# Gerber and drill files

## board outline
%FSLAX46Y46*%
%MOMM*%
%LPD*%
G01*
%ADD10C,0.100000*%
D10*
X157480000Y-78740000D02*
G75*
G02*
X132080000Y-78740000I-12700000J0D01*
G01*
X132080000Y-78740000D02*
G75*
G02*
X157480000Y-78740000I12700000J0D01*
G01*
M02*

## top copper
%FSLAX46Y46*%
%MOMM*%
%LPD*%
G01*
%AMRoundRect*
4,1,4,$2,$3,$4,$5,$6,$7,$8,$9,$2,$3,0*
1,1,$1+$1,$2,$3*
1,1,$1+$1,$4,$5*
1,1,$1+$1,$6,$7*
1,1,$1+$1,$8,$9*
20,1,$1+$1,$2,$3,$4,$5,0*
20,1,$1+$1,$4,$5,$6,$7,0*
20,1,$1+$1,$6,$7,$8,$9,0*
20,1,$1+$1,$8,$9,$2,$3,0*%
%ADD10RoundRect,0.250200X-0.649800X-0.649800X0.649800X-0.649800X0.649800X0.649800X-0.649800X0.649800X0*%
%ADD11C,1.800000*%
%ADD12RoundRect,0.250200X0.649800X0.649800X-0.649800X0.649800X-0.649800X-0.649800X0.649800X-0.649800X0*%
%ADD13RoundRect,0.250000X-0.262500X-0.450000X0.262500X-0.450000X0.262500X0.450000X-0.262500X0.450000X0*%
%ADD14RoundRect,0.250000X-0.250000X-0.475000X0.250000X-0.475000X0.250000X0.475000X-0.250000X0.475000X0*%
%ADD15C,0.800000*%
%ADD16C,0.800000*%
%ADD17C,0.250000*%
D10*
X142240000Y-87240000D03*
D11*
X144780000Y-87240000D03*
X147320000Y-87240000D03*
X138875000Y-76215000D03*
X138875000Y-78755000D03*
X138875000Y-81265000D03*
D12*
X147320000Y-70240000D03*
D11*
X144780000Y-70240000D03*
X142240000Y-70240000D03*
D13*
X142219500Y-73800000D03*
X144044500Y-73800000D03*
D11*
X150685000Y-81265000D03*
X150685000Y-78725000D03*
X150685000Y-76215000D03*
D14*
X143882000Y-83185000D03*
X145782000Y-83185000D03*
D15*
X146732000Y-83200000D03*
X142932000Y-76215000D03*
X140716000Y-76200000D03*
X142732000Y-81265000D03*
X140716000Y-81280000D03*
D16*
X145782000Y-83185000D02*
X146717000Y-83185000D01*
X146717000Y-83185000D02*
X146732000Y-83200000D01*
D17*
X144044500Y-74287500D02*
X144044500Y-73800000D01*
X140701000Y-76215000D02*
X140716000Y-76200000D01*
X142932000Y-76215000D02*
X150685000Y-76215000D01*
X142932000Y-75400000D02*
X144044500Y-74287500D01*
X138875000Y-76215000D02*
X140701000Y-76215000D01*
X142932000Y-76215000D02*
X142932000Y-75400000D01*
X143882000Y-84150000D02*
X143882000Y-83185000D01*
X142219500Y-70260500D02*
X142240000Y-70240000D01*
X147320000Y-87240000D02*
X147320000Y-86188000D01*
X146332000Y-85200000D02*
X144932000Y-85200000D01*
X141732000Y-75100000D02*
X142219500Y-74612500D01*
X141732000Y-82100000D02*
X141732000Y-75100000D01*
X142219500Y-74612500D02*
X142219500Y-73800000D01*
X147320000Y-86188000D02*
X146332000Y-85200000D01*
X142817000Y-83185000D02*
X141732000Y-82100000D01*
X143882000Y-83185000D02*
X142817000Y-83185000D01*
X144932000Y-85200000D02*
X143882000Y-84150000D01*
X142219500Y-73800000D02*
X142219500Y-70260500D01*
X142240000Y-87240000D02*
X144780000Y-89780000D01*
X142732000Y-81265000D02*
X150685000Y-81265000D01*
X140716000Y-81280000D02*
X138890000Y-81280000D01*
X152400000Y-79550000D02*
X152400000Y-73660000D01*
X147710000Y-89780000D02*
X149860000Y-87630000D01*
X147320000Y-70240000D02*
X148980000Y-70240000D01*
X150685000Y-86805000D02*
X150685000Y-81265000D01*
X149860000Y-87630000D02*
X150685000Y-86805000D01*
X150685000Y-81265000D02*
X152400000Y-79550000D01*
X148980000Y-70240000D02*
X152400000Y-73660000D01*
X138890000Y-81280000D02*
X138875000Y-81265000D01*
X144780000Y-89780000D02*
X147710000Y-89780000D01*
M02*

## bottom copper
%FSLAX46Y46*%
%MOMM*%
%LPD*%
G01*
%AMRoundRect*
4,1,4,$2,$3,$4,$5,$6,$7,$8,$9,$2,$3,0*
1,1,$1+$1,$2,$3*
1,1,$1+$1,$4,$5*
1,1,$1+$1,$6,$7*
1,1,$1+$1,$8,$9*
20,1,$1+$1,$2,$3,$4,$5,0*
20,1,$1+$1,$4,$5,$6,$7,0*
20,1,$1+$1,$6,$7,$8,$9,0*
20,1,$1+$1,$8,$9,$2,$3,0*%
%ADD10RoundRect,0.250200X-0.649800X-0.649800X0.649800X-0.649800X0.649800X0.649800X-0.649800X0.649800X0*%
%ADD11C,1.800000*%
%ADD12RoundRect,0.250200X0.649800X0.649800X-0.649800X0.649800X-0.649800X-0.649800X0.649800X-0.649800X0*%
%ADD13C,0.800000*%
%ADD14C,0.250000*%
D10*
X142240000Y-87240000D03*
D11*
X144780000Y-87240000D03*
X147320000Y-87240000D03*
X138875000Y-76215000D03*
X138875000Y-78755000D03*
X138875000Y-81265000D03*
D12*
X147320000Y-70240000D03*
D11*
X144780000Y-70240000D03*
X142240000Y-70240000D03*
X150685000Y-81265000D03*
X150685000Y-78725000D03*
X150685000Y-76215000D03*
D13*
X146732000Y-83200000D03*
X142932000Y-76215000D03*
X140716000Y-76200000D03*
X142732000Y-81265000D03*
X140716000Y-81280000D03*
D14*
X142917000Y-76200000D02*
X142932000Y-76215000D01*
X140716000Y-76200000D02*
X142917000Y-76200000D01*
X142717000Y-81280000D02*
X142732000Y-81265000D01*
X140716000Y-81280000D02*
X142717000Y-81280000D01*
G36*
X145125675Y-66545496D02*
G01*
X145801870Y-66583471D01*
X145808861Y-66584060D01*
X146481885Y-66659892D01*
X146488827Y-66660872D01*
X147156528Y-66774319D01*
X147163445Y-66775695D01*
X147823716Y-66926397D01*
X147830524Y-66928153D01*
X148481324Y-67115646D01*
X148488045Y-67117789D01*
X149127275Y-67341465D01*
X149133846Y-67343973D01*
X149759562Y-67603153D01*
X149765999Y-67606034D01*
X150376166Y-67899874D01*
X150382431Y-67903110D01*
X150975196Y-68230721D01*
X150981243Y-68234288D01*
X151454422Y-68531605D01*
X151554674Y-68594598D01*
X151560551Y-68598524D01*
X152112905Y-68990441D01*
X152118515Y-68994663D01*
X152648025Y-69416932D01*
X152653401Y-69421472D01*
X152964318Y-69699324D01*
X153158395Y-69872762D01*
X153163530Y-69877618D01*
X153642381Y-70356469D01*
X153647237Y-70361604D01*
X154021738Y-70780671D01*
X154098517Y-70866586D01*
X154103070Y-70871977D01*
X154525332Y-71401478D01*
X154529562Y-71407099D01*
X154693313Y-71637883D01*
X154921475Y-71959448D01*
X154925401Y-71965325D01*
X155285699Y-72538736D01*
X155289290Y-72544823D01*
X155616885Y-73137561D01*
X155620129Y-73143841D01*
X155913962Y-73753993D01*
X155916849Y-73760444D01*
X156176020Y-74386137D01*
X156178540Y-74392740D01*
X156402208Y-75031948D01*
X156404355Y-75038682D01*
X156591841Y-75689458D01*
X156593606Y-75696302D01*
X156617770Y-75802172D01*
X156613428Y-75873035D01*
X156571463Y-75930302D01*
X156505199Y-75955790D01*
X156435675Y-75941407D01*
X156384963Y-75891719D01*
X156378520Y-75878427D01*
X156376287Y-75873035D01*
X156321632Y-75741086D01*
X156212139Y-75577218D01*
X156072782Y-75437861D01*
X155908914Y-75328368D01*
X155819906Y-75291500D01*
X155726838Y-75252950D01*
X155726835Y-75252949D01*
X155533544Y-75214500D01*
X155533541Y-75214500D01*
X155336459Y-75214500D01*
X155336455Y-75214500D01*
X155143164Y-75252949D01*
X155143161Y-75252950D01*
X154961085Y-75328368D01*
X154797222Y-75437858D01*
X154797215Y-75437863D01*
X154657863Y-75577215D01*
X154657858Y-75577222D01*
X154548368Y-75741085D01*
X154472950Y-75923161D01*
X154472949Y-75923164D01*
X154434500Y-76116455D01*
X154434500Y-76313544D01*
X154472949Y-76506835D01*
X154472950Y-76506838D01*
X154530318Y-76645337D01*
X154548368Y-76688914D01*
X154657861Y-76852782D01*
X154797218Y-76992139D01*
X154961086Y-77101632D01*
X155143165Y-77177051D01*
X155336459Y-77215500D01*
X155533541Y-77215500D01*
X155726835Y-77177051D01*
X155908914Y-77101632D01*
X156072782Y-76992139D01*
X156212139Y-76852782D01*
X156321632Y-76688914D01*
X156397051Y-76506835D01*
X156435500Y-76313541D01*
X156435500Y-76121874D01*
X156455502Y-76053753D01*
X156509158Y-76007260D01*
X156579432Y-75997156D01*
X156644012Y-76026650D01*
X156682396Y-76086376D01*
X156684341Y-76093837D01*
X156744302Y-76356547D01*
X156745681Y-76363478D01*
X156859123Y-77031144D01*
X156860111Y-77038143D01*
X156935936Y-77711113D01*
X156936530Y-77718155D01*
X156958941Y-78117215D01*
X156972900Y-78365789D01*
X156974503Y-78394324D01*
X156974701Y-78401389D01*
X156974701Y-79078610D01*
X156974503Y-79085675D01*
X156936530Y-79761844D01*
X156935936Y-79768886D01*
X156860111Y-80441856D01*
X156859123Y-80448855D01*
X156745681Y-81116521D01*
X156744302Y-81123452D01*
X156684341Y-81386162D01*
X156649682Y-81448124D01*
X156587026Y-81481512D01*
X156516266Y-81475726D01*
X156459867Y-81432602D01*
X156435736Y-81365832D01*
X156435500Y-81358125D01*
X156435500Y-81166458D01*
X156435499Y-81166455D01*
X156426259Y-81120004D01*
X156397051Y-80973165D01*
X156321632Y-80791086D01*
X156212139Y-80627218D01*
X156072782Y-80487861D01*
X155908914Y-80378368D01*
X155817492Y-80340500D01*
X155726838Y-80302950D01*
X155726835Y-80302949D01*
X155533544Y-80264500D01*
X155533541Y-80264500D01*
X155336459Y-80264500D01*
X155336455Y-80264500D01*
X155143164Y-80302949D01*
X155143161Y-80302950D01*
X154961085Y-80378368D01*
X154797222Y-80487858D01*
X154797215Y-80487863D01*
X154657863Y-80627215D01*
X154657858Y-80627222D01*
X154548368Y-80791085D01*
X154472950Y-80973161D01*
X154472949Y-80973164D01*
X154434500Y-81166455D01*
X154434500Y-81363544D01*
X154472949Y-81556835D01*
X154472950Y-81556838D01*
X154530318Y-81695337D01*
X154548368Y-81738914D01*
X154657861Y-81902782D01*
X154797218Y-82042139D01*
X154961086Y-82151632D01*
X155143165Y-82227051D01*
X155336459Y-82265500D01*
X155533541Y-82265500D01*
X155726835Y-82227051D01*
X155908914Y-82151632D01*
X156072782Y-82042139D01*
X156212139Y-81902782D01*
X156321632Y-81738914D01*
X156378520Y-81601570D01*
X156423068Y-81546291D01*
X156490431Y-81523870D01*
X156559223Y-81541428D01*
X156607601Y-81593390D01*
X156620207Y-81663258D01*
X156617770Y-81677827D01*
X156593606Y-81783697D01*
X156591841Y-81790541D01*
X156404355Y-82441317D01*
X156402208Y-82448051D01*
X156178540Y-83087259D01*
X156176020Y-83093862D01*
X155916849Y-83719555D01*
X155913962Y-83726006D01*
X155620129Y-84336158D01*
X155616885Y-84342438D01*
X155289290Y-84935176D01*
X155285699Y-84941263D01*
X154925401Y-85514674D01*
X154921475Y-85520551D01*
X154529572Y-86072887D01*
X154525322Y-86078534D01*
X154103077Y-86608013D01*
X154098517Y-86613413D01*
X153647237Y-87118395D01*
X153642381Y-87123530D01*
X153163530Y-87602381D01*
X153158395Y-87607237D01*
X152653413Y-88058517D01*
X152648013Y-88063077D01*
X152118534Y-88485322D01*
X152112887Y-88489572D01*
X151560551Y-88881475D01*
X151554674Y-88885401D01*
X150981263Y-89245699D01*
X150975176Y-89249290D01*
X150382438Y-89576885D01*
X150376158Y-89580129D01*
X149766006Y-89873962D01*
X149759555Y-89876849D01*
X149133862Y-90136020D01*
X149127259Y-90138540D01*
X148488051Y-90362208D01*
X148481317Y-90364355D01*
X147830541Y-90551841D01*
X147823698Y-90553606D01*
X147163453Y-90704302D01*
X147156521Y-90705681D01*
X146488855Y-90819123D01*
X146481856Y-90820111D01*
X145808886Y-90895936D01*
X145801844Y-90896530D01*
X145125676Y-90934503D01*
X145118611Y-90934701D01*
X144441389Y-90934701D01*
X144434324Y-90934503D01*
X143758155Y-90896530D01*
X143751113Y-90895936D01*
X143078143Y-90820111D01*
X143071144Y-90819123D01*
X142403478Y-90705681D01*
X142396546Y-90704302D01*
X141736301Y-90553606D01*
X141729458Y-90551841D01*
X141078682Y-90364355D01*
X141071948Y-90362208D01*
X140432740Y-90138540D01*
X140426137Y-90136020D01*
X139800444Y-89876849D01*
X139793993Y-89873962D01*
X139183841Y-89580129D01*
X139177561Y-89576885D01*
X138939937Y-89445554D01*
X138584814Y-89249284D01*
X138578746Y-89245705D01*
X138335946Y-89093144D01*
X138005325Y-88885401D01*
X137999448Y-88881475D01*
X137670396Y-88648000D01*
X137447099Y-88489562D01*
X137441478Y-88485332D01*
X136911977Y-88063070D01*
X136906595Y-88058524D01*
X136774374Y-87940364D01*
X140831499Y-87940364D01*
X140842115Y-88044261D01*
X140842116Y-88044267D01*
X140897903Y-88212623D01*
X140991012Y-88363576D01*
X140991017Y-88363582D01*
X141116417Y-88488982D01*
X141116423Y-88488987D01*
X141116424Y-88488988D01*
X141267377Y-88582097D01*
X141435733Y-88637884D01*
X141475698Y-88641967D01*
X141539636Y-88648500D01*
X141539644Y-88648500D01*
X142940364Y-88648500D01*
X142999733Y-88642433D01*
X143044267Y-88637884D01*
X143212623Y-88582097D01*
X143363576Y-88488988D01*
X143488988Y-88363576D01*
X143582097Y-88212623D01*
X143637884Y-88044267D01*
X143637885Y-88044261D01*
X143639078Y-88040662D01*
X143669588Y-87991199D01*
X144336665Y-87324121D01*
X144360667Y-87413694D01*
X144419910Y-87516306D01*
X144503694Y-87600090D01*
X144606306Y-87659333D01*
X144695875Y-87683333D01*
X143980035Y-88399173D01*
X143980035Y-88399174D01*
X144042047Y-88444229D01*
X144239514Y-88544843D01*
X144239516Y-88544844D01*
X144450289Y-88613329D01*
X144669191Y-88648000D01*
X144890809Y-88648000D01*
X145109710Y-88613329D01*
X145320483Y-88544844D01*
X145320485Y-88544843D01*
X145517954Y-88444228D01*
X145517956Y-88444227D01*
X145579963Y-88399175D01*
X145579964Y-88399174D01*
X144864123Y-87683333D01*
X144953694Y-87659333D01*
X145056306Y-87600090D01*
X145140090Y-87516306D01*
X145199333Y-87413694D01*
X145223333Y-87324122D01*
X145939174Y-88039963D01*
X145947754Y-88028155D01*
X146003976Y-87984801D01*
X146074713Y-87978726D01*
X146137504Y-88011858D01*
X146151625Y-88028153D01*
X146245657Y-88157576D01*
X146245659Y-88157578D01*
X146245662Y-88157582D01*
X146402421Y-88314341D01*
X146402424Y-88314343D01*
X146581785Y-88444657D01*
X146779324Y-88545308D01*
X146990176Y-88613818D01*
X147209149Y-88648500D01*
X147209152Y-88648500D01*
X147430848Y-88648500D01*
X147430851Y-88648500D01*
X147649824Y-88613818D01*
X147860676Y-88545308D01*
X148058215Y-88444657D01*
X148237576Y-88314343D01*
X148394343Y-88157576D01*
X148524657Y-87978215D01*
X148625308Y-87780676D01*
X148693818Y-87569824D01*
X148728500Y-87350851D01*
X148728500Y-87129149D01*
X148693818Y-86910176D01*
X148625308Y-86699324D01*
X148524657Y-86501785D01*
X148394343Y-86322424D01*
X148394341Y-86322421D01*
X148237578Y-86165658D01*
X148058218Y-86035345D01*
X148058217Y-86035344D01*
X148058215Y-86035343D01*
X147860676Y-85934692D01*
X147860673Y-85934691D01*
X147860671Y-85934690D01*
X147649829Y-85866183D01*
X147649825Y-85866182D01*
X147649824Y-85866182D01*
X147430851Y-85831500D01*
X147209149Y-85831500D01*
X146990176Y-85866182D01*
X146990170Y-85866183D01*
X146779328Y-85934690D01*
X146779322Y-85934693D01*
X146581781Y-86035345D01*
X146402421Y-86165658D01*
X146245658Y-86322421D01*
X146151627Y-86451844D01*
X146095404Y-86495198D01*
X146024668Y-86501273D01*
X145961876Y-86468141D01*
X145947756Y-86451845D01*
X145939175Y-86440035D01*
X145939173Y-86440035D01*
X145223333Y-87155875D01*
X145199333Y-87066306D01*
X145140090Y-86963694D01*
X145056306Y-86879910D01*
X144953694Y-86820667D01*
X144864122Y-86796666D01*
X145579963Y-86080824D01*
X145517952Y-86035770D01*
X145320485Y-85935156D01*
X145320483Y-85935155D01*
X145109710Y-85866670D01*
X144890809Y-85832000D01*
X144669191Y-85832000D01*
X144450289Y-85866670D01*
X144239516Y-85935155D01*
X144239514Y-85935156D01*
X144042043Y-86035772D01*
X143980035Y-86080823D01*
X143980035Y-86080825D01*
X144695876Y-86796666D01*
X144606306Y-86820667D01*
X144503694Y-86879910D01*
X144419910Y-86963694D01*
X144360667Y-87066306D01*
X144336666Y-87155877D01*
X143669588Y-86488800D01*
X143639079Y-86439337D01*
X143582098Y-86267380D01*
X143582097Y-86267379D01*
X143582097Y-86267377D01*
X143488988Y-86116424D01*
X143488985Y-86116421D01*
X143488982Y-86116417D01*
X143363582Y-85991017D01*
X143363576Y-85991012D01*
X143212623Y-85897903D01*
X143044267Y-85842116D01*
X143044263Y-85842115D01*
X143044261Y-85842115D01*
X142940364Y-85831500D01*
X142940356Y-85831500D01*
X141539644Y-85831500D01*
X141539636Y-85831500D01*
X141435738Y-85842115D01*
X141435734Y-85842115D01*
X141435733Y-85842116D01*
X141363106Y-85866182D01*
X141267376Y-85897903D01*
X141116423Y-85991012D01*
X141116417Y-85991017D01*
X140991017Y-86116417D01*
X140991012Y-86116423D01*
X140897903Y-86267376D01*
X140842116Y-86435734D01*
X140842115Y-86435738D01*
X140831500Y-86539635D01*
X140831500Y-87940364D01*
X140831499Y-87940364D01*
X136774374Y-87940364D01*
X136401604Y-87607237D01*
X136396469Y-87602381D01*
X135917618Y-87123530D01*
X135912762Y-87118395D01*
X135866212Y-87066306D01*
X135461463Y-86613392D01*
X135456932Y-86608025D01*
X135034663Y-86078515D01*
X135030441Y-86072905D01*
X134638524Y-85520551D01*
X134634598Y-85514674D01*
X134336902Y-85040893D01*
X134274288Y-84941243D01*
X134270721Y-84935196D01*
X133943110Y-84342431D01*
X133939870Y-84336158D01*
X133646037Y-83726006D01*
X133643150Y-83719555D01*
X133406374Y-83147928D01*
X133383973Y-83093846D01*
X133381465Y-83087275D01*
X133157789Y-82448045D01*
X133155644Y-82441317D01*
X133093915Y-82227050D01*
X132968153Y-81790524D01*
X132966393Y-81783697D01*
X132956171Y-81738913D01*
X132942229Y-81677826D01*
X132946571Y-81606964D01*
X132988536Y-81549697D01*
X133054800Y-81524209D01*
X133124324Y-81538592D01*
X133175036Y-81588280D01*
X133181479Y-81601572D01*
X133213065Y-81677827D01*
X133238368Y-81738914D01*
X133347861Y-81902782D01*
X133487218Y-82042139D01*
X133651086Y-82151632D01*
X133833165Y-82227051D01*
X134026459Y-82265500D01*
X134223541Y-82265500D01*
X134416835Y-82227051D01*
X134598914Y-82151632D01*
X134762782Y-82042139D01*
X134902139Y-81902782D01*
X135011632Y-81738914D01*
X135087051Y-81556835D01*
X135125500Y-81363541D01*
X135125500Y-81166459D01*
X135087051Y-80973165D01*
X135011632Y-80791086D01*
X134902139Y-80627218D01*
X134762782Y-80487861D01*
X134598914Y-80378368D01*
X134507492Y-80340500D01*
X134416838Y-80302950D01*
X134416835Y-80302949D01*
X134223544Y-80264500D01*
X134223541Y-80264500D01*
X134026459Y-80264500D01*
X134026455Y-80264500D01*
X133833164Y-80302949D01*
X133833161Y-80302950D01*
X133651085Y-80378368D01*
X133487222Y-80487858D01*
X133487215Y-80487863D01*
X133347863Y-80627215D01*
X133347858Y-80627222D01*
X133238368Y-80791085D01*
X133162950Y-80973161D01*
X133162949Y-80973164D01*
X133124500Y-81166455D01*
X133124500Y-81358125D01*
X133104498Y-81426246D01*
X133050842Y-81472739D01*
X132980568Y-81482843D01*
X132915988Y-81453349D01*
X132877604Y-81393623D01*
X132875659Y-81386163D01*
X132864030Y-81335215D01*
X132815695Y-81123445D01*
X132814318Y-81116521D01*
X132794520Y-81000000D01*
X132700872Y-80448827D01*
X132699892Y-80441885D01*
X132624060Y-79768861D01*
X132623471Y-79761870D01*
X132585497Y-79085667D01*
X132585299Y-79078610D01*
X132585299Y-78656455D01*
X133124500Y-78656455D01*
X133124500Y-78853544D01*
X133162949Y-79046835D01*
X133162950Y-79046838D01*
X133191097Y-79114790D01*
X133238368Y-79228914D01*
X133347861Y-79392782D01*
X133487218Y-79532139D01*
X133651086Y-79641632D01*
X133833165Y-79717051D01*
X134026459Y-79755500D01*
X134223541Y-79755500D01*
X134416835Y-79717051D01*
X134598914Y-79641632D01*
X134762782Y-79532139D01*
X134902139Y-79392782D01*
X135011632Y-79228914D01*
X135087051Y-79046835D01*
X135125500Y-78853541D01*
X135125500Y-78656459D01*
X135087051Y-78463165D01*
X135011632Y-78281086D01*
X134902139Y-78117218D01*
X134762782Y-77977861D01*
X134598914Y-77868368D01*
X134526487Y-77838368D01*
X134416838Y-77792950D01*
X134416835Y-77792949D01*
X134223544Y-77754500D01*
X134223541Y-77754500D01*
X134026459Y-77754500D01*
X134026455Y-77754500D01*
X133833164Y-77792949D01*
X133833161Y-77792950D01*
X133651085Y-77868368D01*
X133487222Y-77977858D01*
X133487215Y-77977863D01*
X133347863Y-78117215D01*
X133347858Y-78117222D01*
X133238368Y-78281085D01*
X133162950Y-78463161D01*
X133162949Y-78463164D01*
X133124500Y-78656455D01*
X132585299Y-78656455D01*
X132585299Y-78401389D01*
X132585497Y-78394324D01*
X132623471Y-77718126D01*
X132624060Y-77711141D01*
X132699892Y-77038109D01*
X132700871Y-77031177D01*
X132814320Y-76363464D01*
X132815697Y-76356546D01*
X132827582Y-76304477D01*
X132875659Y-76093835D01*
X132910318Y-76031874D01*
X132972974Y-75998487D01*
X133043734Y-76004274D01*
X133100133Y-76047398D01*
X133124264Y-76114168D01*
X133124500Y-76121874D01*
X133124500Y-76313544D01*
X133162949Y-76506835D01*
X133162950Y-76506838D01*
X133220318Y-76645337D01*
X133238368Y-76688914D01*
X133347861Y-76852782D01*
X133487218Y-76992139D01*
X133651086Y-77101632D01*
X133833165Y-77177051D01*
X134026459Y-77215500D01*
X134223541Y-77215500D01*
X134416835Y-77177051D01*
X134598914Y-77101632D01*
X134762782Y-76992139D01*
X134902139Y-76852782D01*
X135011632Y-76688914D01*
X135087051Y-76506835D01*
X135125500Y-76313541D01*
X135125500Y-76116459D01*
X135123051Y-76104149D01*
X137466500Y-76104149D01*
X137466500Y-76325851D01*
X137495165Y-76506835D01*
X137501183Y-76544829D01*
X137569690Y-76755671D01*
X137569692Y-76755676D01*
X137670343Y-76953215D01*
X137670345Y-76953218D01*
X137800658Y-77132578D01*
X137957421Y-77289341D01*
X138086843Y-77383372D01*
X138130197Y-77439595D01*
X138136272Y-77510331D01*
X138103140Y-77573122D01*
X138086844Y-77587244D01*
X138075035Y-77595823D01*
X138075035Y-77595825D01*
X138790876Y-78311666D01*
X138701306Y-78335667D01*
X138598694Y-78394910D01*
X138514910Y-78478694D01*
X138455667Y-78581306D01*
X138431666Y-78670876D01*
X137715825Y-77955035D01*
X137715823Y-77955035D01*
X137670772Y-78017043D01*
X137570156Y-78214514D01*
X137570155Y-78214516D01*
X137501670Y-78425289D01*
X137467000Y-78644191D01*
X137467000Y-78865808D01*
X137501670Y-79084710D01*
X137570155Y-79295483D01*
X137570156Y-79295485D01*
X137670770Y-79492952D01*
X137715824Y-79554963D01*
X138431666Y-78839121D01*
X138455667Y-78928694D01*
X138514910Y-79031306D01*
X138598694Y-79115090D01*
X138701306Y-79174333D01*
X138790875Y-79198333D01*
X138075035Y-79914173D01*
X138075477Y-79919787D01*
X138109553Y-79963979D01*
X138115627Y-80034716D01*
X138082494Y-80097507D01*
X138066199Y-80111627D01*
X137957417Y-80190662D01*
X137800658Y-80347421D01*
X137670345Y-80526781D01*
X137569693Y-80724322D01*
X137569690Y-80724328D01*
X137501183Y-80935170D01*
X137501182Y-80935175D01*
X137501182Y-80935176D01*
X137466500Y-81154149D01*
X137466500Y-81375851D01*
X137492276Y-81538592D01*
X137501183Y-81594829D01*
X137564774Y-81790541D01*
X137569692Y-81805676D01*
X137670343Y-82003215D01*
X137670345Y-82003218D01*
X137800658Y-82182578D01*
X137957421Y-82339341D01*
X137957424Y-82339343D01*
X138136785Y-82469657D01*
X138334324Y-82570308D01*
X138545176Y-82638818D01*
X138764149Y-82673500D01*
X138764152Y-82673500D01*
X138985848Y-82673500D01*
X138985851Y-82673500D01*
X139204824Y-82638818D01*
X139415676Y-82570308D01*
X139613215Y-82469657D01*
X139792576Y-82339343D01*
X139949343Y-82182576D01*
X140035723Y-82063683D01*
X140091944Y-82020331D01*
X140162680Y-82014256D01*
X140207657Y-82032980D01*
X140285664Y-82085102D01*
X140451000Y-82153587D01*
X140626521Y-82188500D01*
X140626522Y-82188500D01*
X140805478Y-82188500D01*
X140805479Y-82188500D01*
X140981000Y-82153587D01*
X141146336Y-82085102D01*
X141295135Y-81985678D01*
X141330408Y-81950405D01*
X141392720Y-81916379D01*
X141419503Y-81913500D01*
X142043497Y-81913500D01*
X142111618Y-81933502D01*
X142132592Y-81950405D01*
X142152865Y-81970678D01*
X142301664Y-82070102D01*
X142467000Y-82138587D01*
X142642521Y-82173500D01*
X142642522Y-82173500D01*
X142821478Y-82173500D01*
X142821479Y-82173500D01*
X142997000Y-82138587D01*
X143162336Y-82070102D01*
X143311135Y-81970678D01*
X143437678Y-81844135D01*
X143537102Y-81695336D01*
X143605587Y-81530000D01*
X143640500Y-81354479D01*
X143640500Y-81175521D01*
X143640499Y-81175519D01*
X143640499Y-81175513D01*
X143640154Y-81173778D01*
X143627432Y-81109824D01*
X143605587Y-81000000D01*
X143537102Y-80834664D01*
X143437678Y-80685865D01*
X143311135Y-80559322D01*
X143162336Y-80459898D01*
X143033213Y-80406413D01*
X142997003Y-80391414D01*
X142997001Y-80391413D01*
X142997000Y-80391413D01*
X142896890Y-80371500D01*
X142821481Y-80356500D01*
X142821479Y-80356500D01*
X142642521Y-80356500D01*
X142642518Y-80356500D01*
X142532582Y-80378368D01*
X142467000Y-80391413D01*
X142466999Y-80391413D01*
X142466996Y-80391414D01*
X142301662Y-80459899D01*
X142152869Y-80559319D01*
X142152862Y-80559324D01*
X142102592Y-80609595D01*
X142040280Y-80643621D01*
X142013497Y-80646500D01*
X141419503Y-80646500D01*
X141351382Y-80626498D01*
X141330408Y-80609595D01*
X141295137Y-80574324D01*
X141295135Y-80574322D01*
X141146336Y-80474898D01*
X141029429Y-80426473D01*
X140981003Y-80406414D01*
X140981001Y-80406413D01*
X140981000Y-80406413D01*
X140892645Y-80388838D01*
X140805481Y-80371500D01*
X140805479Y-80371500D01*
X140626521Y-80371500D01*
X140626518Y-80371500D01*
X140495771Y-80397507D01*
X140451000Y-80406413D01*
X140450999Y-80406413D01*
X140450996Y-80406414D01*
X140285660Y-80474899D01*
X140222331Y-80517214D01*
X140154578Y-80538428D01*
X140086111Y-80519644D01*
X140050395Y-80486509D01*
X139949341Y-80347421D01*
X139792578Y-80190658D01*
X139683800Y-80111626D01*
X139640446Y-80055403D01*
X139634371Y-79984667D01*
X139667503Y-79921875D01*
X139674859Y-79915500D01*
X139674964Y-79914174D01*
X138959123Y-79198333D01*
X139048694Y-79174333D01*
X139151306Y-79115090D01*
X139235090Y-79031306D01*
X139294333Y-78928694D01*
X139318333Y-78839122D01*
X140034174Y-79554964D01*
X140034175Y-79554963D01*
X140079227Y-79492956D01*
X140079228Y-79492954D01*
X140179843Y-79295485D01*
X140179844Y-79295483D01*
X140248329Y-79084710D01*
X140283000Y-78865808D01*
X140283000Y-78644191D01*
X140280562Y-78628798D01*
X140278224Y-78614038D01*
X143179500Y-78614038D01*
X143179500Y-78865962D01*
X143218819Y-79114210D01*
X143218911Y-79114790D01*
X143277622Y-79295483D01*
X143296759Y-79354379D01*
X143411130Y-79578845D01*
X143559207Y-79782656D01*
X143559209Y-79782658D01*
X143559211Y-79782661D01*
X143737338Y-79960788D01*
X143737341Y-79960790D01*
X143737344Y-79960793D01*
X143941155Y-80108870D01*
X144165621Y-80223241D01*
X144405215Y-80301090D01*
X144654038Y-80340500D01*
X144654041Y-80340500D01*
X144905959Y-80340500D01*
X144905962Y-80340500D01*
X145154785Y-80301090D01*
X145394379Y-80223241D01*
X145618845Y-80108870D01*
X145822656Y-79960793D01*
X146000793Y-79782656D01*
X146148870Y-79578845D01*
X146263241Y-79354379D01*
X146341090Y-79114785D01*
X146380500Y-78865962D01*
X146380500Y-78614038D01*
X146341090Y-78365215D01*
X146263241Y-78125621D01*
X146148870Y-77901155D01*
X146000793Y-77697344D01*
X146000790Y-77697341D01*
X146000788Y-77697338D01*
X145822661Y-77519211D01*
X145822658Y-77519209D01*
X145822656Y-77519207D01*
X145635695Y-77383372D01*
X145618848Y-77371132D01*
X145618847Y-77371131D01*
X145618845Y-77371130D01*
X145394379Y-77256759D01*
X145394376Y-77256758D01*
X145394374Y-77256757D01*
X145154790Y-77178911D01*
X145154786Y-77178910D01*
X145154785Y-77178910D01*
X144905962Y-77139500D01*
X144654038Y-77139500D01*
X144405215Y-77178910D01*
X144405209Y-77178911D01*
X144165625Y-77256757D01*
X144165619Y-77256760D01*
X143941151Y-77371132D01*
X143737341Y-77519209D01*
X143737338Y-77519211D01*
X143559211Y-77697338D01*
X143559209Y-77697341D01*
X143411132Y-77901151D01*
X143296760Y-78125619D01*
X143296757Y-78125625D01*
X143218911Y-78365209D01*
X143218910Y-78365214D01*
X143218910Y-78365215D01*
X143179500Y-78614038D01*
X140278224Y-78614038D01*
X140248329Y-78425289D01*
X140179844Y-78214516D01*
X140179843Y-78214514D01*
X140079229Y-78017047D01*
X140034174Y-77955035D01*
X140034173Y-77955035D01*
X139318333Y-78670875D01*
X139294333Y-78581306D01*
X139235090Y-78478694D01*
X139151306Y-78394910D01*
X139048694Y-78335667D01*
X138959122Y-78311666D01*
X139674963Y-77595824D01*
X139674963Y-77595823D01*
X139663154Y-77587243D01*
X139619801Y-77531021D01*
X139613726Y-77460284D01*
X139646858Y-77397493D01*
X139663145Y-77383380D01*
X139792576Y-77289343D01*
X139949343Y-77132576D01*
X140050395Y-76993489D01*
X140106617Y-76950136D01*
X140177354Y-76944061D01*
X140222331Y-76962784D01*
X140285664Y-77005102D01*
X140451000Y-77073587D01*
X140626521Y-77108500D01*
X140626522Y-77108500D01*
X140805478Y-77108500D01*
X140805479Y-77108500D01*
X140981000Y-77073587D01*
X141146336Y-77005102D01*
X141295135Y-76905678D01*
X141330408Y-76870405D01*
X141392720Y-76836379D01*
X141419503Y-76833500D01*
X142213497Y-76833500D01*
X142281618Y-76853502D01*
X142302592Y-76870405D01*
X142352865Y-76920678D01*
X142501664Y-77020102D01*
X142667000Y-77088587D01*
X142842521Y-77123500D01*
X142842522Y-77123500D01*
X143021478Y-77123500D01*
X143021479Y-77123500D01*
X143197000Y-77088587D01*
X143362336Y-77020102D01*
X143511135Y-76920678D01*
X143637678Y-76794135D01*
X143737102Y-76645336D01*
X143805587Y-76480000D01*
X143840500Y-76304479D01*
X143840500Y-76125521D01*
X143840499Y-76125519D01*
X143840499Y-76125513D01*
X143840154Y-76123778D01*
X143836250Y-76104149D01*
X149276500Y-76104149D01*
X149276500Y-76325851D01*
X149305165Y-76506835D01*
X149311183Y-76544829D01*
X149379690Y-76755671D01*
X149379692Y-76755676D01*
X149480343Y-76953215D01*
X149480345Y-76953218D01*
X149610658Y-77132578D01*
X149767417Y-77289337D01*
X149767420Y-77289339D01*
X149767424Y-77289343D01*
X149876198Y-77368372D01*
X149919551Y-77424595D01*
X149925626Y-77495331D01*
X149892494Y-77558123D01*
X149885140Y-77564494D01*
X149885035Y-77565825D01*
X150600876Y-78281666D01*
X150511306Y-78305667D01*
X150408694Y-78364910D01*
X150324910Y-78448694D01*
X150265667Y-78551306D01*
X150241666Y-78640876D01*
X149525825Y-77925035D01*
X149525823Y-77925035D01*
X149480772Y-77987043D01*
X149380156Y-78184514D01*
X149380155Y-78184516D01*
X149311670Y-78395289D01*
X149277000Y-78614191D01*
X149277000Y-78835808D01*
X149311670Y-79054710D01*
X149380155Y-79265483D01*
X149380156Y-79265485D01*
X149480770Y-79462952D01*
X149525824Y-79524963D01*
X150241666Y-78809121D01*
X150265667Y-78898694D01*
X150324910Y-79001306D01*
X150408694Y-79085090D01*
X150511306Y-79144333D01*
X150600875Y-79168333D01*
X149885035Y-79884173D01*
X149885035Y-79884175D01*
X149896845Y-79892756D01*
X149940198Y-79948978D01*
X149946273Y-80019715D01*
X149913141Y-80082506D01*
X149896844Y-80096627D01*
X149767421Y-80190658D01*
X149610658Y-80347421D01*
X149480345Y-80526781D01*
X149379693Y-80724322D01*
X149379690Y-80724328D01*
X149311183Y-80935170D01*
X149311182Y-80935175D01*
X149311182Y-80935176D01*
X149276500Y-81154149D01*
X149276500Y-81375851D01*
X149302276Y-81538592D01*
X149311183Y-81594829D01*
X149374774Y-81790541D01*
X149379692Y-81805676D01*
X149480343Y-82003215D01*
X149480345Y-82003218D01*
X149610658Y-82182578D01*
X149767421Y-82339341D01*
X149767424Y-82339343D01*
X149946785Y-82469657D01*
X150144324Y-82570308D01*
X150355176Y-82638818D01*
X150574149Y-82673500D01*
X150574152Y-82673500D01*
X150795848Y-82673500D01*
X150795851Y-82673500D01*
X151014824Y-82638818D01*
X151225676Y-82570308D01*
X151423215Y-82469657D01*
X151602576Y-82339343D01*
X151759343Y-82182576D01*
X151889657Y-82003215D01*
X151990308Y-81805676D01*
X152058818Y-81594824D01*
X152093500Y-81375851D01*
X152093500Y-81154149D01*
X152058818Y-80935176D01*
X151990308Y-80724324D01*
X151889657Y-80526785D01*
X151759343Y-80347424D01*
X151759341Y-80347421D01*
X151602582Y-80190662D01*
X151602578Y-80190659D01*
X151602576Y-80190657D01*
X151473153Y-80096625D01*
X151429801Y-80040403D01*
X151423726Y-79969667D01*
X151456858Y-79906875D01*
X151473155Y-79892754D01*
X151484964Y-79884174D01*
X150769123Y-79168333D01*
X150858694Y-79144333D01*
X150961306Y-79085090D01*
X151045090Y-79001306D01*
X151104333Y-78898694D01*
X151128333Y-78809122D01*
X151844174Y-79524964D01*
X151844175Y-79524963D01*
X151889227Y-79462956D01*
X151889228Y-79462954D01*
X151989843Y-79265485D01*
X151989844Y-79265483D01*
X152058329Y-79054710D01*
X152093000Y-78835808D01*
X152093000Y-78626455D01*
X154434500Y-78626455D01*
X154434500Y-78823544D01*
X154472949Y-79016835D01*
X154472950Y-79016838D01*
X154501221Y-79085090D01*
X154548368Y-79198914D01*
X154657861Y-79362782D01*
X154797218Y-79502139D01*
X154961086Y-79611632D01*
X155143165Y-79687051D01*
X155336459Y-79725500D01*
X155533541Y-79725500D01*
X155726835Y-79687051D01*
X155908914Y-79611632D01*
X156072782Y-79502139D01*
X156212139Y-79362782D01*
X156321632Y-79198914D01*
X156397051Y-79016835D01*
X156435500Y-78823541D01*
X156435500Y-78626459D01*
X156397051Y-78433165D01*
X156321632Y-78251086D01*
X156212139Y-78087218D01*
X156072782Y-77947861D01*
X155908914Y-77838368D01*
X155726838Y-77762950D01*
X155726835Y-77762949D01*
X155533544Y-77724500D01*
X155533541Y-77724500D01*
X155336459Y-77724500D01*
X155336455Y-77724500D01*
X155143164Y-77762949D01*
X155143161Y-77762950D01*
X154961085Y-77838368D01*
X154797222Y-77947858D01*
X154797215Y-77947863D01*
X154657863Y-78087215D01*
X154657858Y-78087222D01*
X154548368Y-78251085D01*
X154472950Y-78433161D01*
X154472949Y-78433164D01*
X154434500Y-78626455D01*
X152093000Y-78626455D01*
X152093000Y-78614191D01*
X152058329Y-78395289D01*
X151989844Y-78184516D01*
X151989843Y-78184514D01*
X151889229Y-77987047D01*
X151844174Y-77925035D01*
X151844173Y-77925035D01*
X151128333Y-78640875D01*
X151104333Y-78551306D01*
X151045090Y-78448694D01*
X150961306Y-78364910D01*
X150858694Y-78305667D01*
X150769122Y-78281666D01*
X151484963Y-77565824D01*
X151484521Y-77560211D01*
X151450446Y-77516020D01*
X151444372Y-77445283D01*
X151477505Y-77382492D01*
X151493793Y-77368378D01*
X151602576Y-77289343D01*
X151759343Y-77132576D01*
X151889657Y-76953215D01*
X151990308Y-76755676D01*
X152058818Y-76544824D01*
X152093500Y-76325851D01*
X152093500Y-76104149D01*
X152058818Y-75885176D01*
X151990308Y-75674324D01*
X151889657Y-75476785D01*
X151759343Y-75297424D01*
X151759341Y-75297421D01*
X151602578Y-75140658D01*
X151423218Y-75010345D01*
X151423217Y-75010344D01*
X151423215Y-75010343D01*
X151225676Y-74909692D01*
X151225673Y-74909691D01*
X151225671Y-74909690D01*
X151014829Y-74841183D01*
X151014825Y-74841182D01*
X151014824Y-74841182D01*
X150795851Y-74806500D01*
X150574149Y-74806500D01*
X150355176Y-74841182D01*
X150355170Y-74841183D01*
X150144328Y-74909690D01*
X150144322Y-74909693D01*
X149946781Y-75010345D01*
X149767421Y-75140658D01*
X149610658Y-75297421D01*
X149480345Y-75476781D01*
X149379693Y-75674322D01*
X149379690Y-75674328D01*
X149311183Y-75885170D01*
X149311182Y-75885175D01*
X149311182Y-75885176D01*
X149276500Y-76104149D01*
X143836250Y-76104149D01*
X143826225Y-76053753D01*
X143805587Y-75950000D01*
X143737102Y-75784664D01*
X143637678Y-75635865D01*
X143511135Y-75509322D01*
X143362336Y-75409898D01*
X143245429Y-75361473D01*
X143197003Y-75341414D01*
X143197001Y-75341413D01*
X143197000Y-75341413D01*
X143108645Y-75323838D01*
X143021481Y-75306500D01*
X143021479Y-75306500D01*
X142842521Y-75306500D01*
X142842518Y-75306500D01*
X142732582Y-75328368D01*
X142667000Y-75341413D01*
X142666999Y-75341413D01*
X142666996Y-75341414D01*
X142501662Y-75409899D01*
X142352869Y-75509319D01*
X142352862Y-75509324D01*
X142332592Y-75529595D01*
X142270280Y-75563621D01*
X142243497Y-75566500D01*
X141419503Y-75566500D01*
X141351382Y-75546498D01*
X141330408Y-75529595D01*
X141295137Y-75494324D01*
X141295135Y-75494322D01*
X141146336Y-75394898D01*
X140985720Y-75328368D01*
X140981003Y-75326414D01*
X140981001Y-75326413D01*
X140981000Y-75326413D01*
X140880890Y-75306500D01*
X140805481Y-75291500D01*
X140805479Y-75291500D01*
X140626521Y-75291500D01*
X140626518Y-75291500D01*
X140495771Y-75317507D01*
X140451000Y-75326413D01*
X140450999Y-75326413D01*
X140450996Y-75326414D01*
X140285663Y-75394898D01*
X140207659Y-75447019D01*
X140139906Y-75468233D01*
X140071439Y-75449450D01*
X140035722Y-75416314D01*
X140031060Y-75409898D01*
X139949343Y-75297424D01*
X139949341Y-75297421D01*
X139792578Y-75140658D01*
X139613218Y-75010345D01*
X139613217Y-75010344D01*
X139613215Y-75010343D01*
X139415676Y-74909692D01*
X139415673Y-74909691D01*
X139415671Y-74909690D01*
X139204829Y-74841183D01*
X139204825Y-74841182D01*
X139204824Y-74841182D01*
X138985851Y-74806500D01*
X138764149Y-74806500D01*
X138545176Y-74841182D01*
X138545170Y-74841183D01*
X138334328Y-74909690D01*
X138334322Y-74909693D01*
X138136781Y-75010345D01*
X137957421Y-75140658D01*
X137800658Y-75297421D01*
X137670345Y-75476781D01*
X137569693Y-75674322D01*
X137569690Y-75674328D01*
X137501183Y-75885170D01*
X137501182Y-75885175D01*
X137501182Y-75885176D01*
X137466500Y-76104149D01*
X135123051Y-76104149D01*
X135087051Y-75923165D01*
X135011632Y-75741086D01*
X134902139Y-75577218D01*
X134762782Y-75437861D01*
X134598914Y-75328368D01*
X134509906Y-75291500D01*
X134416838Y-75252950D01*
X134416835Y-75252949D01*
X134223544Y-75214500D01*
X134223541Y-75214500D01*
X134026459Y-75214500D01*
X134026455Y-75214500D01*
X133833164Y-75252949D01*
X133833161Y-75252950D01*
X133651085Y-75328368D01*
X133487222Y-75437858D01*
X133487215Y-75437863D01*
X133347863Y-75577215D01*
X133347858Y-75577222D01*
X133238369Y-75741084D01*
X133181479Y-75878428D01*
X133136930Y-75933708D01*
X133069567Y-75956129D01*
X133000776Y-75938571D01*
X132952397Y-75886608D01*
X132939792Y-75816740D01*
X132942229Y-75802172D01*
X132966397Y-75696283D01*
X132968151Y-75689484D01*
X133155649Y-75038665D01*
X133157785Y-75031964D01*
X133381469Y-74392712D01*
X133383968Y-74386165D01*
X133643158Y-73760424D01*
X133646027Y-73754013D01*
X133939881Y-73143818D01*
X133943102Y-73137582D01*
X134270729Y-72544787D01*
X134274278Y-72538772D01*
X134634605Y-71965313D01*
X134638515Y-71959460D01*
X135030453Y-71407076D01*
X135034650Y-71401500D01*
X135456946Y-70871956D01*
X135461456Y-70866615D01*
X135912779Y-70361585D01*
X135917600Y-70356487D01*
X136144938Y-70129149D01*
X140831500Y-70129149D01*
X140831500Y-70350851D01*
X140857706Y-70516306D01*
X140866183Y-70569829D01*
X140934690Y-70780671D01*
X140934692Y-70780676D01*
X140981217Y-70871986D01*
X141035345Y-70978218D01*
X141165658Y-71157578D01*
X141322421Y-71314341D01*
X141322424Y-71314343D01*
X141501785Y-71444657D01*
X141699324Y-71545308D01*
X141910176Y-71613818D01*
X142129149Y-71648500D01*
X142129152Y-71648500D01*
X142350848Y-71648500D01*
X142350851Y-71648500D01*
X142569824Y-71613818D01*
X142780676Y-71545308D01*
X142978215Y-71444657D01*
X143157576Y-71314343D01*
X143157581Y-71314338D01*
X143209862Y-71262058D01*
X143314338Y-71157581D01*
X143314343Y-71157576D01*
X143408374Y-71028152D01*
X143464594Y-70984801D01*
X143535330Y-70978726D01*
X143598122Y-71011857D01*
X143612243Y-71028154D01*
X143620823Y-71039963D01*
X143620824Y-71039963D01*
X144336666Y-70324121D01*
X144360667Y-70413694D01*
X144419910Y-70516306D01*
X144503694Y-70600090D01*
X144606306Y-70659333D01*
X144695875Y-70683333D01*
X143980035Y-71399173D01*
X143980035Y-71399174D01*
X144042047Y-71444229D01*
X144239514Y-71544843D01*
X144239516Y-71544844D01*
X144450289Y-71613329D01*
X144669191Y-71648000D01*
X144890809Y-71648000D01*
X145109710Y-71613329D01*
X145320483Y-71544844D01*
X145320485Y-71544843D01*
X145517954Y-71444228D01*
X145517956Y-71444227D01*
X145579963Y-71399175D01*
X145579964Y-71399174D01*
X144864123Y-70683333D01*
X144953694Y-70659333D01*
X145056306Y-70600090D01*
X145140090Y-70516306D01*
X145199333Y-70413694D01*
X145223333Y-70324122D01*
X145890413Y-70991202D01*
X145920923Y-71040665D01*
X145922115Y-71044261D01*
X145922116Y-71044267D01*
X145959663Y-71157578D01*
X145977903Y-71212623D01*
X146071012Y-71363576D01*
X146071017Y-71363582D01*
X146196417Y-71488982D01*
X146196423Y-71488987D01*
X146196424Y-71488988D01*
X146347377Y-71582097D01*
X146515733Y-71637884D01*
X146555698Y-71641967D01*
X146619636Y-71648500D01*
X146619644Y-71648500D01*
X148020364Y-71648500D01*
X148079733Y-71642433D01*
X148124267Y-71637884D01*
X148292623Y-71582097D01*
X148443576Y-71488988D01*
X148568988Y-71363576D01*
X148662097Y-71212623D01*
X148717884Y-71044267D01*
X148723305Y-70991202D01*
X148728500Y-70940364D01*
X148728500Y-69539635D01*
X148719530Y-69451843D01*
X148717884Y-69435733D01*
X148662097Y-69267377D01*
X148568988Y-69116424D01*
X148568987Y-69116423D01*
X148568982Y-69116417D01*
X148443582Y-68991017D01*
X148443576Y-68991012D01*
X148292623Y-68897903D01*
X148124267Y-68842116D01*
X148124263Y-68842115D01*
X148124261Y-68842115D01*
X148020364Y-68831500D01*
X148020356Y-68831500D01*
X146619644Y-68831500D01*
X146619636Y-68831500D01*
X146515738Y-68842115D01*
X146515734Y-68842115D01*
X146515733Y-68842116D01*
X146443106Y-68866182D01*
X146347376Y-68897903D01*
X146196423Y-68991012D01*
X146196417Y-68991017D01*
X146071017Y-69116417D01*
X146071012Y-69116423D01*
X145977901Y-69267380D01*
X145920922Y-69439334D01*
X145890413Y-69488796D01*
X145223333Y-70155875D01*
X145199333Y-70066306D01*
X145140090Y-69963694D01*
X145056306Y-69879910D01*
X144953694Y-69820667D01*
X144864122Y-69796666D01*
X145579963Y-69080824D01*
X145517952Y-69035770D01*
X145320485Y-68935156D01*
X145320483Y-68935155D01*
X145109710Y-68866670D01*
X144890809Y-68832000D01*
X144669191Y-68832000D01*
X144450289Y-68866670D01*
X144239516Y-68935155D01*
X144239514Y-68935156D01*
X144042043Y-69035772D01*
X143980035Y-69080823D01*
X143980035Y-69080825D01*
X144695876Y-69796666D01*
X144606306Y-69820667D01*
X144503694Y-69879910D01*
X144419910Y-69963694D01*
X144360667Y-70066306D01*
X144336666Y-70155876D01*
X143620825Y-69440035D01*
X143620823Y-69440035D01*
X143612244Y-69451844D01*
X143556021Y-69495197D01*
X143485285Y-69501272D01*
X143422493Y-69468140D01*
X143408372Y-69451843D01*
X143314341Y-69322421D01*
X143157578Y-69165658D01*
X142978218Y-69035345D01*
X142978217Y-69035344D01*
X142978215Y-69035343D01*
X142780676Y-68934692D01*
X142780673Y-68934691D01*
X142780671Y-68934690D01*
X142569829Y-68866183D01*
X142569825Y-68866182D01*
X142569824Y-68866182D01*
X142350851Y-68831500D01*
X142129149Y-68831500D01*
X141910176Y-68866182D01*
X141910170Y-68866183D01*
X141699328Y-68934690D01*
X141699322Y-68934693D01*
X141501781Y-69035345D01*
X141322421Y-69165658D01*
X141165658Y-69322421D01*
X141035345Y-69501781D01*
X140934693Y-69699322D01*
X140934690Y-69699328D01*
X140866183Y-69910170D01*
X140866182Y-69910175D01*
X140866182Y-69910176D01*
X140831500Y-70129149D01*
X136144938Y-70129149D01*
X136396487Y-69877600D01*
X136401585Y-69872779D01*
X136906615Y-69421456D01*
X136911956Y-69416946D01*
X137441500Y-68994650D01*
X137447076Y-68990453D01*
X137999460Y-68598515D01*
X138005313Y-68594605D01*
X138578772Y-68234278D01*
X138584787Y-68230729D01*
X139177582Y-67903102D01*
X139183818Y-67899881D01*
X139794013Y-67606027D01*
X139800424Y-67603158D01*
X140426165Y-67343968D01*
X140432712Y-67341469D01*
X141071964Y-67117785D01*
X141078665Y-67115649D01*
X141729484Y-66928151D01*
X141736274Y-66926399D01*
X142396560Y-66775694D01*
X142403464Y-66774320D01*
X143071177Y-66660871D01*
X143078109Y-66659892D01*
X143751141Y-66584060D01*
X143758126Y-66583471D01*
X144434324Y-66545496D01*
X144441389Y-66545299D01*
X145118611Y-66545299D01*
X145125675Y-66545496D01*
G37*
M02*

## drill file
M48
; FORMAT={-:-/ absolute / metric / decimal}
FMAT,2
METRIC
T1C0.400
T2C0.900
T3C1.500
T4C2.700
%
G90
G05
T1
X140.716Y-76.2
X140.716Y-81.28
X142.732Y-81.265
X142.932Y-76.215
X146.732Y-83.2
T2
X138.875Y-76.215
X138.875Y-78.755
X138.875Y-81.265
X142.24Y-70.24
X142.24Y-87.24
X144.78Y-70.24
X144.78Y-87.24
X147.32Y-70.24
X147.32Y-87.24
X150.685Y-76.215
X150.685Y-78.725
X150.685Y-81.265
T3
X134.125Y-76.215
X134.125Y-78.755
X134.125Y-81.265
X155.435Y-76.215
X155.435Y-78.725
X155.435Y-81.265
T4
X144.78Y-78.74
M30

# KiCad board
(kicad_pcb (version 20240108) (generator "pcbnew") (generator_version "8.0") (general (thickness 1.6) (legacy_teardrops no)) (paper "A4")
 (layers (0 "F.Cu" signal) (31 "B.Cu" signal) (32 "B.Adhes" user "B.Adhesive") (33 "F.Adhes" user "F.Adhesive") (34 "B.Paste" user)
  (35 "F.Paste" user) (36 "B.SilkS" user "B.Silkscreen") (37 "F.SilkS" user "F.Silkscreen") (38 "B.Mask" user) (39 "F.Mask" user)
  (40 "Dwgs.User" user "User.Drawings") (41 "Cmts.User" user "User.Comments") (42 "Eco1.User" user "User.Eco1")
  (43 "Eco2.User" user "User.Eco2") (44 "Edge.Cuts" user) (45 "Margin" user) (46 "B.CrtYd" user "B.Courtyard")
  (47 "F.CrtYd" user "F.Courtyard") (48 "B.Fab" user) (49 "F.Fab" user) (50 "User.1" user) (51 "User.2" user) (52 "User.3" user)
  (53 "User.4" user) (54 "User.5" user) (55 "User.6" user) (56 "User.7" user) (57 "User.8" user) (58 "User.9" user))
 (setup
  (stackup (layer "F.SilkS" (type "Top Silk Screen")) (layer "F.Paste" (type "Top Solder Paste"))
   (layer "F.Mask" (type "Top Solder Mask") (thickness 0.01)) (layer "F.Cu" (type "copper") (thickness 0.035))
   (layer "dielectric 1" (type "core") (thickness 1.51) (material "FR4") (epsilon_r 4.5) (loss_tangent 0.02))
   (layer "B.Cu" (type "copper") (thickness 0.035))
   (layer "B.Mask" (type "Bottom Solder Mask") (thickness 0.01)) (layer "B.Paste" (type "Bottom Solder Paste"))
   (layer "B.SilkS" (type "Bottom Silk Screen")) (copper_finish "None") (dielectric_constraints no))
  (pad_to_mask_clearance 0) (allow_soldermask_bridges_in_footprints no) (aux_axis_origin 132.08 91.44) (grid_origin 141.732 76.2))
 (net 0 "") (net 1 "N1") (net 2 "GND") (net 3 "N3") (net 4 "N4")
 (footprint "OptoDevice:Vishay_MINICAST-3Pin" (layer "F.Cu") (at 142.24 87.24)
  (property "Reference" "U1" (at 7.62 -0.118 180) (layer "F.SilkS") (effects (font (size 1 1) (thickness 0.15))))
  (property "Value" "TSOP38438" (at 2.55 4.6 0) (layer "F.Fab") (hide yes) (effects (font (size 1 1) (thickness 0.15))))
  (pad "1" thru_hole roundrect (at 0 0) (size 1.8 1.8) (drill 0.9) (layers "*.Cu" "*.Mask") (remove_unused_layers no)
   (roundrect_rratio 0.139) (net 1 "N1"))
  (pad "2" thru_hole circle (at 2.54 0) (size 1.8 1.8) (drill 0.9) (layers "*.Cu" "*.Mask") (remove_unused_layers no) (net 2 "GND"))
  (pad "3" thru_hole circle (at 5.08 0) (size 1.8 1.8) (drill 0.9) (layers "*.Cu" "*.Mask") (remove_unused_layers no) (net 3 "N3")))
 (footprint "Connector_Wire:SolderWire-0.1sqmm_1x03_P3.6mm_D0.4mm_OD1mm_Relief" (layer "F.Cu") (at 138.875 75.155 -90)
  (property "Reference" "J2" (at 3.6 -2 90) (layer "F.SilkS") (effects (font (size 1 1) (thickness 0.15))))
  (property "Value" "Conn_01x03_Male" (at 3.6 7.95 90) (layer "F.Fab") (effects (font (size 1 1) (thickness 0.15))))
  (pad "" np_thru_hole circle (at 1.06 4.75 270) (size 1.5 1.5) (drill 1.5) (layers "*.Cu" "*.Mask"))
  (pad "" np_thru_hole circle (at 3.6 4.75 270) (size 1.5 1.5) (drill 1.5) (layers "*.Cu" "*.Mask"))
  (pad "" np_thru_hole circle (at 6.11 4.75 270) (size 1.5 1.5) (drill 1.5) (layers "*.Cu" "*.Mask"))
  (pad "1" thru_hole circle (at 1.06 0 270) (size 1.8 1.8) (drill 0.9) (layers "*.Cu" "*.Mask") (remove_unused_layers no) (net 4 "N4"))
  (pad "2" thru_hole circle (at 3.6 0 270) (size 1.8 1.8) (drill 0.9) (layers "*.Cu" "*.Mask") (remove_unused_layers no) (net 2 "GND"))
  (pad "3" thru_hole circle (at 6.11 0 270) (size 1.8 1.8) (drill 0.9) (layers "*.Cu" "*.Mask") (remove_unused_layers no) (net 1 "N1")))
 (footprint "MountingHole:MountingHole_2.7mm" (layer "F.Cu") (at 144.78 78.74)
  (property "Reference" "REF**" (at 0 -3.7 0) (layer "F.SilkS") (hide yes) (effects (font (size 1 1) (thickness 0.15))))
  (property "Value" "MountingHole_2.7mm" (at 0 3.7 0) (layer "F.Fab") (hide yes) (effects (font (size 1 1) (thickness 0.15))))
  (pad "" np_thru_hole circle (at 0 0) (size 2.7 2.7) (drill 2.7) (layers "*.Cu" "*.Mask")))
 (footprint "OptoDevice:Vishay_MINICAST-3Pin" (layer "F.Cu") (at 147.32 70.24 180)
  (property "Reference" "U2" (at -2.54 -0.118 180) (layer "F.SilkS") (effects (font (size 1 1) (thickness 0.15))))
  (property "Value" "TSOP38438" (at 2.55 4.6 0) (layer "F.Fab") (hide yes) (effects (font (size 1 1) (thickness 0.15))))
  (pad "1" thru_hole roundrect (at 0 0 180) (size 1.8 1.8) (drill 0.9) (layers "*.Cu" "*.Mask") (remove_unused_layers no)
   (roundrect_rratio 0.139) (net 1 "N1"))
  (pad "2" thru_hole circle (at 2.54 0 180) (size 1.8 1.8) (drill 0.9) (layers "*.Cu" "*.Mask") (remove_unused_layers no) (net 2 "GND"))
  (pad "3" thru_hole circle (at 5.08 0 180) (size 1.8 1.8) (drill 0.9) (layers "*.Cu" "*.Mask") (remove_unused_layers no) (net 3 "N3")))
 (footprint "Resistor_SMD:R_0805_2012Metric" (layer "F.Cu") (at 143.132 73.8)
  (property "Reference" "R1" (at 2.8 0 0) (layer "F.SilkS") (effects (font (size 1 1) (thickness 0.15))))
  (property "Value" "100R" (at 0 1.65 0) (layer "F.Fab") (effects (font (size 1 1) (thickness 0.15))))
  (pad "1" smd roundrect (at -0.9125 0) (size 1.025 1.4) (layers "F.Cu" "F.Paste" "F.Mask") (roundrect_rratio 0.243902) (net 3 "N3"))
  (pad "2" smd roundrect (at 0.9125 0) (size 1.025 1.4) (layers "F.Cu" "F.Paste" "F.Mask") (roundrect_rratio 0.243902) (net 4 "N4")))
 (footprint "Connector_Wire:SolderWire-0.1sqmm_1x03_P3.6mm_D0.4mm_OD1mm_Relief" (layer "F.Cu") (at 150.685 81.265 90)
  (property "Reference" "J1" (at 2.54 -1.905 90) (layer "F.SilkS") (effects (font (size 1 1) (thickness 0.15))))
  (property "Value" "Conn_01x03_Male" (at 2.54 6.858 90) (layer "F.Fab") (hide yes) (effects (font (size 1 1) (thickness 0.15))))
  (pad "" np_thru_hole circle (at 0 4.75 90) (size 1.5 1.5) (drill 1.5) (layers "*.Cu" "*.Mask"))
  (pad "" np_thru_hole circle (at 2.54 4.75 90) (size 1.5 1.5) (drill 1.5) (layers "*.Cu" "*.Mask"))
  (pad "" np_thru_hole circle (at 5.05 4.75 90) (size 1.5 1.5) (drill 1.5) (layers "*.Cu" "*.Mask"))
  (pad "1" thru_hole circle (at 0 0 90) (size 1.8 1.8) (drill 0.9) (layers "*.Cu" "*.Mask") (remove_unused_layers no) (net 1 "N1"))
  (pad "2" thru_hole circle (at 2.54 0 90) (size 1.8 1.8) (drill 0.9) (layers "*.Cu" "*.Mask") (remove_unused_layers no) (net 2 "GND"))
  (pad "3" thru_hole circle (at 5.05 0 90) (size 1.8 1.8) (drill 0.9) (layers "*.Cu" "*.Mask") (remove_unused_layers no) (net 4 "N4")))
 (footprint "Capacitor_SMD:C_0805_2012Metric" (layer "F.Cu") (at 144.832 83.185)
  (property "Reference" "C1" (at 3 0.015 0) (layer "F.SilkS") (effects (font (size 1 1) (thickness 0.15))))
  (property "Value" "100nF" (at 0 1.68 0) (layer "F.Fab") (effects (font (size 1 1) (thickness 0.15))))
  (pad "1" smd roundrect (at -0.95 0) (size 1 1.45) (layers "F.Cu" "F.Paste" "F.Mask") (roundrect_rratio 0.25) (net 3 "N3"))
  (pad "2" smd roundrect (at 0.95 0) (size 1 1.45) (layers "F.Cu" "F.Paste" "F.Mask") (roundrect_rratio 0.25) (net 2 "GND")))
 (gr_circle (center 144.78 78.74) (end 157.48 78.74) (stroke (width 0.1) (type solid)) (fill none) (layer "Edge.Cuts"))
 (segment (start 145.782 83.185) (end 146.717 83.185) (width 0.8) (layer "F.Cu") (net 2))
 (segment (start 146.717 83.185) (end 146.732 83.2) (width 0.8) (layer "F.Cu") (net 2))
 (via (at 146.732 83.2) (size 0.8) (drill 0.4) (layers "F.Cu" "B.Cu") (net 2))
 (segment (start 144.0445 74.2875) (end 144.0445 73.8) (width 0.25) (layer "F.Cu") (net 4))
 (segment (start 140.701 76.215) (end 140.716 76.2) (width 0.25) (layer "F.Cu") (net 4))
 (segment (start 142.932 76.215) (end 150.685 76.215) (width 0.25) (layer "F.Cu") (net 4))
 (segment (start 142.932 75.4) (end 144.0445 74.2875) (width 0.25) (layer "F.Cu") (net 4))
 (segment (start 138.875 76.215) (end 140.701 76.215) (width 0.25) (layer "F.Cu") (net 4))
 (segment (start 142.932 76.215) (end 142.932 75.4) (width 0.25) (layer "F.Cu") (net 4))
 (via (at 142.932 76.215) (size 0.8) (drill 0.4) (layers "F.Cu" "B.Cu") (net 4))
 (via (at 140.716 76.2) (size 0.8) (drill 0.4) (layers "F.Cu" "B.Cu") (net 4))
 (segment (start 142.917 76.2) (end 142.932 76.215) (width 0.25) (layer "B.Cu") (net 4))
 (segment (start 140.716 76.2) (end 142.917 76.2) (width 0.25) (layer "B.Cu") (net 4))
 (segment (start 143.882 84.15) (end 143.882 83.185) (width 0.25) (layer "F.Cu") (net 3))
 (segment (start 142.2195 70.2605) (end 142.24 70.24) (width 0.25) (layer "F.Cu") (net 3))
 (segment (start 147.32 87.24) (end 147.32 86.188) (width 0.25) (layer "F.Cu") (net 3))
 (segment (start 146.332 85.2) (end 144.932 85.2) (width 0.25) (layer "F.Cu") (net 3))
 (segment (start 141.732 75.1) (end 142.2195 74.6125) (width 0.25) (layer "F.Cu") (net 3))
 (segment (start 141.732 82.1) (end 141.732 75.1) (width 0.25) (layer "F.Cu") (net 3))
 (segment (start 142.2195 74.6125) (end 142.2195 73.8) (width 0.25) (layer "F.Cu") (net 3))
 (segment (start 147.32 86.188) (end 146.332 85.2) (width 0.25) (layer "F.Cu") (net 3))
 (segment (start 142.817 83.185) (end 141.732 82.1) (width 0.25) (layer "F.Cu") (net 3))
 (segment (start 143.882 83.185) (end 142.817 83.185) (width 0.25) (layer "F.Cu") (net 3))
 (segment (start 144.932 85.2) (end 143.882 84.15) (width 0.25) (layer "F.Cu") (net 3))
 (segment (start 142.2195 73.8) (end 142.2195 70.2605) (width 0.25) (layer "F.Cu") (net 3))
 (segment (start 142.24 87.24) (end 144.78 89.78) (width 0.25) (layer "F.Cu") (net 1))
 (segment (start 142.732 81.265) (end 150.685 81.265) (width 0.25) (layer "F.Cu") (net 1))
 (segment (start 140.716 81.28) (end 138.89 81.28) (width 0.25) (layer "F.Cu") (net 1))
 (segment (start 152.4 79.55) (end 152.4 73.66) (width 0.25) (layer "F.Cu") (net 1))
 (segment (start 147.71 89.78) (end 149.86 87.63) (width 0.25) (layer "F.Cu") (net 1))
 (segment (start 147.32 70.24) (end 148.98 70.24) (width 0.25) (layer "F.Cu") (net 1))
 (segment (start 150.685 86.805) (end 150.685 81.265) (width 0.25) (layer "F.Cu") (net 1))
 (segment (start 149.86 87.63) (end 150.685 86.805) (width 0.25) (layer "F.Cu") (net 1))
 (segment (start 150.685 81.265) (end 152.4 79.55) (width 0.25) (layer "F.Cu") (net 1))
 (segment (start 148.98 70.24) (end 152.4 73.66) (width 0.25) (layer "F.Cu") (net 1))
 (segment (start 138.89 81.28) (end 138.875 81.265) (width 0.25) (layer "F.Cu") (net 1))
 (segment (start 144.78 89.78) (end 147.71 89.78) (width 0.25) (layer "F.Cu") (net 1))
 (via (at 142.732 81.265) (size 0.8) (drill 0.4) (layers "F.Cu" "B.Cu") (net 1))
 (via (at 140.716 81.28) (size 0.8) (drill 0.4) (layers "F.Cu" "B.Cu") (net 1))
 (segment (start 142.717 81.28) (end 142.732 81.265) (width 0.25) (layer "B.Cu") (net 1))
 (segment (start 140.716 81.28) (end 142.717 81.28) (width 0.25) (layer "B.Cu") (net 1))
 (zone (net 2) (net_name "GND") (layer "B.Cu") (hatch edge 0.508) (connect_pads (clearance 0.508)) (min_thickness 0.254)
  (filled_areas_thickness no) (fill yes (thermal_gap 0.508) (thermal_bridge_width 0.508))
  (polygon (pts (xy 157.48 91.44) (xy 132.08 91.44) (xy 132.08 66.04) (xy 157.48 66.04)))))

